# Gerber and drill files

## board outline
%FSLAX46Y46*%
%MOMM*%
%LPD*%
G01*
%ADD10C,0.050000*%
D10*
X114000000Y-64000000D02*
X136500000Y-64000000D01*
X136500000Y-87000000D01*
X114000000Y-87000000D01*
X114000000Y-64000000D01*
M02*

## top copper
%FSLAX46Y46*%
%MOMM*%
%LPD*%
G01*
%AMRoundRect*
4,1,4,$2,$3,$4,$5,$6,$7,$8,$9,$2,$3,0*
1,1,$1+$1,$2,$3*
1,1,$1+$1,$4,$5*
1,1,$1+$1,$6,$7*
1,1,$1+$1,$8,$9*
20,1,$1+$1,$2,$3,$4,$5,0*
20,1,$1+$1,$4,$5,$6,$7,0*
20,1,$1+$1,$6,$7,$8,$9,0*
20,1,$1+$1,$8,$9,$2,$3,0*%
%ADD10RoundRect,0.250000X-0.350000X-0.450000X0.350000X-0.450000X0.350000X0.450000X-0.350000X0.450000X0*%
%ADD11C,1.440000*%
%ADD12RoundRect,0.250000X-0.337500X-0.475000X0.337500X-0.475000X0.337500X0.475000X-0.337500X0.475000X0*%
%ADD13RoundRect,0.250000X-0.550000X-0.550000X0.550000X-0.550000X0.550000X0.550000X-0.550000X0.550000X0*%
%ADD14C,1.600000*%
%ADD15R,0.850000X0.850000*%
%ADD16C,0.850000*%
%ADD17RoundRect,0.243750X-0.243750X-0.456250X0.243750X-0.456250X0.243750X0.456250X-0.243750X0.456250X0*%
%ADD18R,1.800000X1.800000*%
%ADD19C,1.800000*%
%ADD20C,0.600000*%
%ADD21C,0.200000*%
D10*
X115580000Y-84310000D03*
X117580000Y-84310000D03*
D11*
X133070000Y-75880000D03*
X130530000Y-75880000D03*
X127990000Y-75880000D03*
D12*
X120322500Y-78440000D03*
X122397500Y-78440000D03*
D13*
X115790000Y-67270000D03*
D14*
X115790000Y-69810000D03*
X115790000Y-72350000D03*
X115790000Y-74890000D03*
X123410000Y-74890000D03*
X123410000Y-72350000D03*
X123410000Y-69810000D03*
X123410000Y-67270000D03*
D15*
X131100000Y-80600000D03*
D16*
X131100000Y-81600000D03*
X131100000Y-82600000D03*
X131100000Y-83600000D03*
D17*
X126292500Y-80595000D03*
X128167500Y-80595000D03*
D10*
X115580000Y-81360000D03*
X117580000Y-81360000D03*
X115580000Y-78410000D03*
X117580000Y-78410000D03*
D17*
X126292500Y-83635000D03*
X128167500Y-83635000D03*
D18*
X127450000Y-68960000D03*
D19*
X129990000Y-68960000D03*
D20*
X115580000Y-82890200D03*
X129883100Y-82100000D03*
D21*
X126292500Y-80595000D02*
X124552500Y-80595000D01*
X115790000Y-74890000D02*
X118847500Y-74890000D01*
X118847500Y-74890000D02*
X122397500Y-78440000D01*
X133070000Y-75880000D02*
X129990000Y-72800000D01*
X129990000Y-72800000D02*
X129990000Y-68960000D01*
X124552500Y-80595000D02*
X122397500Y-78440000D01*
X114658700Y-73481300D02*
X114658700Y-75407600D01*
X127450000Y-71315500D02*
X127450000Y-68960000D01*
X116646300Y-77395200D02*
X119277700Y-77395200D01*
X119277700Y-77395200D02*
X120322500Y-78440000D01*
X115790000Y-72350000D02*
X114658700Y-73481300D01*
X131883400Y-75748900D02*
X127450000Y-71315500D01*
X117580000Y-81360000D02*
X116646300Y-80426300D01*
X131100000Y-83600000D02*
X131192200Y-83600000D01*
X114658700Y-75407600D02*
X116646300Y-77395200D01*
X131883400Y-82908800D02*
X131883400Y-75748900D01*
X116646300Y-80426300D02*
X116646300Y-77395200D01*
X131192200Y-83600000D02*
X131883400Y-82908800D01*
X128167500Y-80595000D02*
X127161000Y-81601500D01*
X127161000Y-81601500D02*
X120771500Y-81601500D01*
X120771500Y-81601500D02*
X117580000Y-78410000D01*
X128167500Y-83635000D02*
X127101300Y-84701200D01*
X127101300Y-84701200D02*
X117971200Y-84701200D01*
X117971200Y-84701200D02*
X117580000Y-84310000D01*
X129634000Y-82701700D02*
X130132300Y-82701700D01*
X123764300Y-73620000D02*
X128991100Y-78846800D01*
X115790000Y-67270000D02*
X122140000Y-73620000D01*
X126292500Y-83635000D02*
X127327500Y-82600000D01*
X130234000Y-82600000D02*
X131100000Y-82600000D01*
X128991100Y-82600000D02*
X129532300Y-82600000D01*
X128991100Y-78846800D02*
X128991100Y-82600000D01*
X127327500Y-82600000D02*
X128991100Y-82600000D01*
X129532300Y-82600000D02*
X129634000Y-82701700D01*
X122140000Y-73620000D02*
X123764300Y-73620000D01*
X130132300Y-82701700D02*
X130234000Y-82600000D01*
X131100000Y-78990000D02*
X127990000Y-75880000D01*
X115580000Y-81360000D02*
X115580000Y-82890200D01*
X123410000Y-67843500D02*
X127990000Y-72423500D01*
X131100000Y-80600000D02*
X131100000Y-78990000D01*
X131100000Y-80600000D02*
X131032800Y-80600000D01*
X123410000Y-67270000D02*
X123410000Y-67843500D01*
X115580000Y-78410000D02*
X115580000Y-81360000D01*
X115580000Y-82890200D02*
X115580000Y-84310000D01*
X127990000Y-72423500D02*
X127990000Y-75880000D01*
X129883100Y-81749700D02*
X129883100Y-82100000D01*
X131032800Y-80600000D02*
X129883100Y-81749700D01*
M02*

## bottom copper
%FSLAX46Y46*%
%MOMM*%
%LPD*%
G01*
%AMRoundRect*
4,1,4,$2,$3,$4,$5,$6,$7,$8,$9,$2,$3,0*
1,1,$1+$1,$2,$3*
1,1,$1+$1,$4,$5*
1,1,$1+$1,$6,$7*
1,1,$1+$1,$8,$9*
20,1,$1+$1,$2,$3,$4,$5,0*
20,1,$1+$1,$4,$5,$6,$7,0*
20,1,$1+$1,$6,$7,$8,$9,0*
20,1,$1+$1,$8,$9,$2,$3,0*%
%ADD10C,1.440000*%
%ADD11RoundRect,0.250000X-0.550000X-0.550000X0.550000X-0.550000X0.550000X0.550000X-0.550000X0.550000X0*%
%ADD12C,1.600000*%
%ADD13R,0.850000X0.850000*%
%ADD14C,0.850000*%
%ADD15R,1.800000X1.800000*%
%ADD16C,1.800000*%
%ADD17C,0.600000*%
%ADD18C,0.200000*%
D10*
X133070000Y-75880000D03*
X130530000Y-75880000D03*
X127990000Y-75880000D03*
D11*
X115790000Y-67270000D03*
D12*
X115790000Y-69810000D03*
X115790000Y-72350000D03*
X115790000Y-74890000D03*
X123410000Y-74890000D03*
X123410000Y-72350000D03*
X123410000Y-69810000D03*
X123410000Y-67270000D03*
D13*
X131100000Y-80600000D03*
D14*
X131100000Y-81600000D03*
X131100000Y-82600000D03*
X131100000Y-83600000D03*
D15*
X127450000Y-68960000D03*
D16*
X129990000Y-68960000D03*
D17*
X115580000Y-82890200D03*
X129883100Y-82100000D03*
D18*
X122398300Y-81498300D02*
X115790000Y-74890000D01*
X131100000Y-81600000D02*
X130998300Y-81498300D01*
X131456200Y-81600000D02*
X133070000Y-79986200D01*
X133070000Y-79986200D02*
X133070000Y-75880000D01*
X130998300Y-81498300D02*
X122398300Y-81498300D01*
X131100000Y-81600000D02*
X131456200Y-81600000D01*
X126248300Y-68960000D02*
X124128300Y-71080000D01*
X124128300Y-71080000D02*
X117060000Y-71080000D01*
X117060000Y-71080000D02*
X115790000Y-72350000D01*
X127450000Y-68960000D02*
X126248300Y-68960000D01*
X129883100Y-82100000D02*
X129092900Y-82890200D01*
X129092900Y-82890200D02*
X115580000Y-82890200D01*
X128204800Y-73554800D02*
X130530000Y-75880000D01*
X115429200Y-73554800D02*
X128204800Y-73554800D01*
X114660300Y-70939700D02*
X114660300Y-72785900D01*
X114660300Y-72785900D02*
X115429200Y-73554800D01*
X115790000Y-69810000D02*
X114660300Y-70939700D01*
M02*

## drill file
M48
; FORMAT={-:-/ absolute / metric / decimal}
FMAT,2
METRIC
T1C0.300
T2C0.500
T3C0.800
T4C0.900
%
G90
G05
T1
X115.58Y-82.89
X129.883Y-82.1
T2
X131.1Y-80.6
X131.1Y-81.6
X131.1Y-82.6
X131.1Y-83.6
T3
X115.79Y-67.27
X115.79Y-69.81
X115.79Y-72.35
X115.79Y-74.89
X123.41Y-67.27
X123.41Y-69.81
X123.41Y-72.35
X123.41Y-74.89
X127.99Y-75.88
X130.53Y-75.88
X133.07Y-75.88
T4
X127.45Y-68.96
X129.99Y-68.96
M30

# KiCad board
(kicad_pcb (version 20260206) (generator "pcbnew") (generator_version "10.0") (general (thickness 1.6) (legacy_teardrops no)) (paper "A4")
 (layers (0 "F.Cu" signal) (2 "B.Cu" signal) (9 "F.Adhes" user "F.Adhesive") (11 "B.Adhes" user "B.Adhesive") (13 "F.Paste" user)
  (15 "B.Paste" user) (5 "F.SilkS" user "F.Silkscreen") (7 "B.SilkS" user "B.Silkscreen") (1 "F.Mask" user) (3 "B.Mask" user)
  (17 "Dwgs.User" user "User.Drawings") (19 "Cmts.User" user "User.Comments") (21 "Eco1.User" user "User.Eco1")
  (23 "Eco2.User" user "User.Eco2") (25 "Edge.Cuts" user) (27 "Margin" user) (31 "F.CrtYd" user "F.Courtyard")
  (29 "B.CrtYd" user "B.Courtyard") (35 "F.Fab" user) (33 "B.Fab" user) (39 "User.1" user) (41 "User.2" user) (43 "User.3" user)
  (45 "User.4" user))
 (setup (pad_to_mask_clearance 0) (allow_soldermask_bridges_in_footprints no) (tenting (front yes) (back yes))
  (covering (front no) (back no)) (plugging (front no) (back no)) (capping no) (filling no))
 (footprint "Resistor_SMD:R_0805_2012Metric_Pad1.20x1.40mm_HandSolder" (layer "F.Cu") (at 116.58 84.31)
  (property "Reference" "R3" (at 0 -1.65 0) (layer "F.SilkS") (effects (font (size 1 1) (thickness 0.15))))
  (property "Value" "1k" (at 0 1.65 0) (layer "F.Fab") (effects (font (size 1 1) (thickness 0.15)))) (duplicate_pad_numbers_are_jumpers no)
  (pad "1" smd roundrect (at -1 0) (size 1.2 1.4) (layers "F.Cu" "F.Mask" "F.Paste") (roundrect_rratio 0.208333) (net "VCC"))
  (pad "2" smd roundrect (at 1 0) (size 1.2 1.4) (layers "F.Cu" "F.Mask" "F.Paste") (roundrect_rratio 0.208333) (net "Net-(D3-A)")))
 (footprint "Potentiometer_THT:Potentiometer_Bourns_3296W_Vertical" (layer "F.Cu") (at 133.07 75.88)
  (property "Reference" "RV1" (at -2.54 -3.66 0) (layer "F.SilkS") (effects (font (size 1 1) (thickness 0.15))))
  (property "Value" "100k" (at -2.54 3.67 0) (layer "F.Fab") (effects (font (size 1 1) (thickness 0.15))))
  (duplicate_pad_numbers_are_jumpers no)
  (pad "1" thru_hole circle (at 0 0) (size 1.44 1.44) (drill 0.8) (layers "*.Cu" "*.Mask") (remove_unused_layers no) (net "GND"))
  (pad "2" thru_hole circle (at -2.54 0) (size 1.44 1.44) (drill 0.8) (layers "*.Cu" "*.Mask") (remove_unused_layers no) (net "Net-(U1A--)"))
  (pad "3" thru_hole circle (at -5.08 0) (size 1.44 1.44) (drill 0.8) (layers "*.Cu" "*.Mask") (remove_unused_layers no) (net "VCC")))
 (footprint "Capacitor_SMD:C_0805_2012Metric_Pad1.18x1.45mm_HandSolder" (layer "F.Cu") (at 121.36 78.44)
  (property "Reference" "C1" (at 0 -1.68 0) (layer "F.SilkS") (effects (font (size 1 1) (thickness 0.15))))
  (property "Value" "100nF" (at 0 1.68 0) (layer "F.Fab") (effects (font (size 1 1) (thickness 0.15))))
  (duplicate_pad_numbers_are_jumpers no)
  (pad "1" smd roundrect (at -1.0375 0) (size 1.175 1.45) (layers "F.Cu" "F.Mask" "F.Paste") (roundrect_rratio 0.212766) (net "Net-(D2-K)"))
  (pad "2" smd roundrect (at 1.0375 0) (size 1.175 1.45) (layers "F.Cu" "F.Mask" "F.Paste") (roundrect_rratio 0.212766) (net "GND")))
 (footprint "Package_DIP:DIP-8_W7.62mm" (layer "F.Cu") (at 115.79 67.27)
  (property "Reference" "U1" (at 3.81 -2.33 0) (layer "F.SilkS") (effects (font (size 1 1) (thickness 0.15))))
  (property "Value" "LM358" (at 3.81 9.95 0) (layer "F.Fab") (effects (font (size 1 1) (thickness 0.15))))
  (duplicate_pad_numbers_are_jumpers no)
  (pad "1" thru_hole roundrect (at 0 0) (size 1.6 1.6) (drill 0.8) (layers "*.Cu" "*.Mask") (remove_unused_layers no)
   (roundrect_rratio 0.15625) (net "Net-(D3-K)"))
  (pad "2" thru_hole circle (at 0 2.54) (size 1.6 1.6) (drill 0.8) (layers "*.Cu" "*.Mask") (remove_unused_layers no) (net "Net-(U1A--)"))
  (pad "3" thru_hole circle (at 0 5.08) (size 1.6 1.6) (drill 0.8) (layers "*.Cu" "*.Mask") (remove_unused_layers no) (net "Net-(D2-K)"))
  (pad "4" thru_hole circle (at 0 7.62) (size 1.6 1.6) (drill 0.8) (layers "*.Cu" "*.Mask") (remove_unused_layers no) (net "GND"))
  (pad "5" thru_hole circle (at 7.62 7.62) (size 1.6 1.6) (drill 0.8) (layers "*.Cu" "*.Mask") (remove_unused_layers no)
   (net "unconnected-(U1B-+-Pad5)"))
  (pad "6" thru_hole circle (at 7.62 5.08) (size 1.6 1.6) (drill 0.8) (layers "*.Cu" "*.Mask") (remove_unused_layers no)
   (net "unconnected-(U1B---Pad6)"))
  (pad "7" thru_hole circle (at 7.62 2.54) (size 1.6 1.6) (drill 0.8) (layers "*.Cu" "*.Mask") (remove_unused_layers no)
   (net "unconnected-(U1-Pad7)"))
  (pad "8" thru_hole circle (at 7.62 0) (size 1.6 1.6) (drill 0.8) (layers "*.Cu" "*.Mask") (remove_unused_layers no) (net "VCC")))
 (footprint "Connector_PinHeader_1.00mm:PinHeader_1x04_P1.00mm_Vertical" (layer "F.Cu") (at 131.1 80.6)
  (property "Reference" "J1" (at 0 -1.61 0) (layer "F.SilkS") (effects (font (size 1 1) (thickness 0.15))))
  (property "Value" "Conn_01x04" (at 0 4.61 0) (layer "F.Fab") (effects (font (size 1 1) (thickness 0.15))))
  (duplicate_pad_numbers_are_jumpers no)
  (pad "1" thru_hole rect (at 0 0) (size 0.85 0.85) (drill 0.5) (layers "*.Cu" "*.Mask") (remove_unused_layers no) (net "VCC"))
  (pad "2" thru_hole circle (at 0 1) (size 0.85 0.85) (drill 0.5) (layers "*.Cu" "*.Mask") (remove_unused_layers no) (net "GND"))
  (pad "3" thru_hole circle (at 0 2) (size 0.85 0.85) (drill 0.5) (layers "*.Cu" "*.Mask") (remove_unused_layers no) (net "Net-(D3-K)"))
  (pad "4" thru_hole circle (at 0 3) (size 0.85 0.85) (drill 0.5) (layers "*.Cu" "*.Mask") (remove_unused_layers no) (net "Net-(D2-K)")))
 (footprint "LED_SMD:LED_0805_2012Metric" (layer "F.Cu") (at 127.23 80.595)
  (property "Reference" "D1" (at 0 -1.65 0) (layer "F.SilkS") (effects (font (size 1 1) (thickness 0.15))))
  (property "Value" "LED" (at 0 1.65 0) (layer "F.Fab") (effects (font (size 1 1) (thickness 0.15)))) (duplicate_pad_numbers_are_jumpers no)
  (pad "1" smd roundrect (at -0.9375 0) (size 0.975 1.4) (layers "F.Cu" "F.Mask" "F.Paste") (roundrect_rratio 0.25) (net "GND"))
  (pad "2" smd roundrect (at 0.9375 0) (size 0.975 1.4) (layers "F.Cu" "F.Mask" "F.Paste") (roundrect_rratio 0.25) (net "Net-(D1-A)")))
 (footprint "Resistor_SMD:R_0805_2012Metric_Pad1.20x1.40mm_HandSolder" (layer "F.Cu") (at 116.58 81.36)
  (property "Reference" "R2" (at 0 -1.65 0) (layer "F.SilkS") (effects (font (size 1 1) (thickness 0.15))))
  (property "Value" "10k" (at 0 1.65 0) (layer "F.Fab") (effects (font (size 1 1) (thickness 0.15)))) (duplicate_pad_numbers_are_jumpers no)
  (pad "1" smd roundrect (at -1 0) (size 1.2 1.4) (layers "F.Cu" "F.Mask" "F.Paste") (roundrect_rratio 0.208333) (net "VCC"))
  (pad "2" smd roundrect (at 1 0) (size 1.2 1.4) (layers "F.Cu" "F.Mask" "F.Paste") (roundrect_rratio 0.208333) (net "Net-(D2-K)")))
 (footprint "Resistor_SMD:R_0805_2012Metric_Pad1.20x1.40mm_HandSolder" (layer "F.Cu") (at 116.58 78.41)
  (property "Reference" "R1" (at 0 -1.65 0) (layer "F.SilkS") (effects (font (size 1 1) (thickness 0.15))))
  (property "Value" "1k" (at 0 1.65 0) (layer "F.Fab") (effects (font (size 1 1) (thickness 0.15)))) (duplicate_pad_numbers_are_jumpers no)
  (pad "1" smd roundrect (at -1 0) (size 1.2 1.4) (layers "F.Cu" "F.Mask" "F.Paste") (roundrect_rratio 0.208333) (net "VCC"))
  (pad "2" smd roundrect (at 1 0) (size 1.2 1.4) (layers "F.Cu" "F.Mask" "F.Paste") (roundrect_rratio 0.208333) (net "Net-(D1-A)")))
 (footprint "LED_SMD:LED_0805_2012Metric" (layer "F.Cu") (at 127.23 83.635)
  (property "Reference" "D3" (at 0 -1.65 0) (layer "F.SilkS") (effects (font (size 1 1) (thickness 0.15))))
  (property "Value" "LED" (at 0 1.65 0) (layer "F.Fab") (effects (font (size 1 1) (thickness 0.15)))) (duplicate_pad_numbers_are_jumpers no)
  (pad "1" smd roundrect (at -0.9375 0) (size 0.975 1.4) (layers "F.Cu" "F.Mask" "F.Paste") (roundrect_rratio 0.25) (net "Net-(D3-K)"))
  (pad "2" smd roundrect (at 0.9375 0) (size 0.975 1.4) (layers "F.Cu" "F.Mask" "F.Paste") (roundrect_rratio 0.25) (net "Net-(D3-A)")))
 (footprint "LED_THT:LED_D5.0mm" (layer "F.Cu") (at 127.45 68.96)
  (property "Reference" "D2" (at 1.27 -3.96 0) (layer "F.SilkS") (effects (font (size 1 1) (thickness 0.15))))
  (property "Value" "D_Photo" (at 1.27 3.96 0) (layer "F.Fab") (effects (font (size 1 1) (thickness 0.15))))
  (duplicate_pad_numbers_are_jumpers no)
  (pad "1" thru_hole rect (at 0 0) (size 1.8 1.8) (drill 0.9) (layers "*.Cu" "*.Mask") (remove_unused_layers no) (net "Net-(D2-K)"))
  (pad "2" thru_hole circle (at 2.54 0) (size 1.8 1.8) (drill 0.9) (layers "*.Cu" "*.Mask") (remove_unused_layers no) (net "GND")))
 (gr_rect (start 114 64) (end 136.5 87) (stroke (width 0.05) (type default)) (fill no) (layer "Edge.Cuts"))
 (segment (start 126.2925 80.595) (end 124.5525 80.595) (width 0.2) (layer "F.Cu") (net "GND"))
 (segment (start 115.79 74.89) (end 118.8475 74.89) (width 0.2) (layer "F.Cu") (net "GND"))
 (segment (start 118.8475 74.89) (end 122.3975 78.44) (width 0.2) (layer "F.Cu") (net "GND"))
 (segment (start 133.07 75.88) (end 129.99 72.8) (width 0.2) (layer "F.Cu") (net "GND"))
 (segment (start 129.99 72.8) (end 129.99 68.96) (width 0.2) (layer "F.Cu") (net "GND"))
 (segment (start 124.5525 80.595) (end 122.3975 78.44) (width 0.2) (layer "F.Cu") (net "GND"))
 (segment (start 122.3983 81.4983) (end 115.79 74.89) (width 0.2) (layer "B.Cu") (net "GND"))
 (segment (start 131.1 81.6) (end 130.9983 81.4983) (width 0.2) (layer "B.Cu") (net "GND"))
 (segment (start 131.4562 81.6) (end 133.07 79.9862) (width 0.2) (layer "B.Cu") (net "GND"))
 (segment (start 133.07 79.9862) (end 133.07 75.88) (width 0.2) (layer "B.Cu") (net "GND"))
 (segment (start 130.9983 81.4983) (end 122.3983 81.4983) (width 0.2) (layer "B.Cu") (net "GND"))
 (segment (start 131.1 81.6) (end 131.4562 81.6) (width 0.2) (layer "B.Cu") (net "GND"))
 (segment (start 114.6587 73.4813) (end 114.6587 75.4076) (width 0.2) (layer "F.Cu") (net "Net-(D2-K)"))
 (segment (start 127.45 71.3155) (end 127.45 68.96) (width 0.2) (layer "F.Cu") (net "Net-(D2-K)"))
 (segment (start 116.6463 77.3952) (end 119.2777 77.3952) (width 0.2) (layer "F.Cu") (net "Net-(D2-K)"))
 (segment (start 119.2777 77.3952) (end 120.3225 78.44) (width 0.2) (layer "F.Cu") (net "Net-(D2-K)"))
 (segment (start 115.79 72.35) (end 114.6587 73.4813) (width 0.2) (layer "F.Cu") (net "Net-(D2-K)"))
 (segment (start 131.8834 75.7489) (end 127.45 71.3155) (width 0.2) (layer "F.Cu") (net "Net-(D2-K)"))
 (segment (start 117.58 81.36) (end 116.6463 80.4263) (width 0.2) (layer "F.Cu") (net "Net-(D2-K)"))
 (segment (start 131.1 83.6) (end 131.1922 83.6) (width 0.2) (layer "F.Cu") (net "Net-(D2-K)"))
 (segment (start 114.6587 75.4076) (end 116.6463 77.3952) (width 0.2) (layer "F.Cu") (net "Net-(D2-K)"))
 (segment (start 131.8834 82.9088) (end 131.8834 75.7489) (width 0.2) (layer "F.Cu") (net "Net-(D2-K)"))
 (segment (start 116.6463 80.4263) (end 116.6463 77.3952) (width 0.2) (layer "F.Cu") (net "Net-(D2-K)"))
 (segment (start 131.1922 83.6) (end 131.8834 82.9088) (width 0.2) (layer "F.Cu") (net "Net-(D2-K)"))
 (segment (start 126.2483 68.96) (end 124.1283 71.08) (width 0.2) (layer "B.Cu") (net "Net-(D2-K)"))
 (segment (start 124.1283 71.08) (end 117.06 71.08) (width 0.2) (layer "B.Cu") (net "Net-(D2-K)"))
 (segment (start 117.06 71.08) (end 115.79 72.35) (width 0.2) (layer "B.Cu") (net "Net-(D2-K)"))
 (segment (start 127.45 68.96) (end 126.2483 68.96) (width 0.2) (layer "B.Cu") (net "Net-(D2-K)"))
 (segment (start 128.1675 80.595) (end 127.161 81.6015) (width 0.2) (layer "F.Cu") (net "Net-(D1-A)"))
 (segment (start 127.161 81.6015) (end 120.7715 81.6015) (width 0.2) (layer "F.Cu") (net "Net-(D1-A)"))
 (segment (start 120.7715 81.6015) (end 117.58 78.41) (width 0.2) (layer "F.Cu") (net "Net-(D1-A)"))
 (segment (start 128.1675 83.635) (end 127.1013 84.7012) (width 0.2) (layer "F.Cu") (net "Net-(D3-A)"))
 (segment (start 127.1013 84.7012) (end 117.9712 84.7012) (width 0.2) (layer "F.Cu") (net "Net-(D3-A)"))
 (segment (start 117.9712 84.7012) (end 117.58 84.31) (width 0.2) (layer "F.Cu") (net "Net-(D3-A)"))
 (segment (start 129.634 82.7017) (end 130.1323 82.7017) (width 0.2) (layer "F.Cu") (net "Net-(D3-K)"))
 (segment (start 123.7643 73.62) (end 128.9911 78.8468) (width 0.2) (layer "F.Cu") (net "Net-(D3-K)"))
 (segment (start 115.79 67.27) (end 122.14 73.62) (width 0.2) (layer "F.Cu") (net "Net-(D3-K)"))
 (segment (start 126.2925 83.635) (end 127.3275 82.6) (width 0.2) (layer "F.Cu") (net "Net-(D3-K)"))
 (segment (start 130.234 82.6) (end 131.1 82.6) (width 0.2) (layer "F.Cu") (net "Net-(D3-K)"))
 (segment (start 128.9911 82.6) (end 129.5323 82.6) (width 0.2) (layer "F.Cu") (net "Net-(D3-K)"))
 (segment (start 128.9911 78.8468) (end 128.9911 82.6) (width 0.2) (layer "F.Cu") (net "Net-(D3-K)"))
 (segment (start 127.3275 82.6) (end 128.9911 82.6) (width 0.2) (layer "F.Cu") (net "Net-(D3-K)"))
 (segment (start 129.5323 82.6) (end 129.634 82.7017) (width 0.2) (layer "F.Cu") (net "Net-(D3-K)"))
 (segment (start 122.14 73.62) (end 123.7643 73.62) (width 0.2) (layer "F.Cu") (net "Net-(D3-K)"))
 (segment (start 130.1323 82.7017) (end 130.234 82.6) (width 0.2) (layer "F.Cu") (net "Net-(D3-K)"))
 (segment (start 131.1 78.99) (end 127.99 75.88) (width 0.2) (layer "F.Cu") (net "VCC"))
 (segment (start 115.58 81.36) (end 115.58 82.8902) (width 0.2) (layer "F.Cu") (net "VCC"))
 (segment (start 123.41 67.8435) (end 127.99 72.4235) (width 0.2) (layer "F.Cu") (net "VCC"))
 (segment (start 131.1 80.6) (end 131.1 78.99) (width 0.2) (layer "F.Cu") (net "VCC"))
 (segment (start 131.1 80.6) (end 131.0328 80.6) (width 0.2) (layer "F.Cu") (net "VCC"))
 (segment (start 123.41 67.27) (end 123.41 67.8435) (width 0.2) (layer "F.Cu") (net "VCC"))
 (segment (start 115.58 78.41) (end 115.58 81.36) (width 0.2) (layer "F.Cu") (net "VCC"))
 (segment (start 115.58 82.8902) (end 115.58 84.31) (width 0.2) (layer "F.Cu") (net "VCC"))
 (segment (start 127.99 72.4235) (end 127.99 75.88) (width 0.2) (layer "F.Cu") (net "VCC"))
 (segment (start 129.8831 81.7497) (end 129.8831 82.1) (width 0.2) (layer "F.Cu") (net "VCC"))
 (segment (start 131.0328 80.6) (end 129.8831 81.7497) (width 0.2) (layer "F.Cu") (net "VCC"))
 (via (at 115.58 82.8902) (size 0.6) (drill 0.3) (layers "F.Cu" "B.Cu") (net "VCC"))
 (via (at 129.8831 82.1) (size 0.6) (drill 0.3) (layers "F.Cu" "B.Cu") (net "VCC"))
 (segment (start 129.8831 82.1) (end 129.0929 82.8902) (width 0.2) (layer "B.Cu") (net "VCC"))
 (segment (start 129.0929 82.8902) (end 115.58 82.8902) (width 0.2) (layer "B.Cu") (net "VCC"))
 (segment (start 128.2048 73.5548) (end 130.53 75.88) (width 0.2) (layer "B.Cu") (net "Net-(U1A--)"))
 (segment (start 115.4292 73.5548) (end 128.2048 73.5548) (width 0.2) (layer "B.Cu") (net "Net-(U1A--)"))
 (segment (start 114.6603 70.9397) (end 114.6603 72.7859) (width 0.2) (layer "B.Cu") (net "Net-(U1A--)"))
 (segment (start 114.6603 72.7859) (end 115.4292 73.5548) (width 0.2) (layer "B.Cu") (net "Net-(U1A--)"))
 (segment (start 115.79 69.81) (end 114.6603 70.9397) (width 0.2) (layer "B.Cu") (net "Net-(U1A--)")))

